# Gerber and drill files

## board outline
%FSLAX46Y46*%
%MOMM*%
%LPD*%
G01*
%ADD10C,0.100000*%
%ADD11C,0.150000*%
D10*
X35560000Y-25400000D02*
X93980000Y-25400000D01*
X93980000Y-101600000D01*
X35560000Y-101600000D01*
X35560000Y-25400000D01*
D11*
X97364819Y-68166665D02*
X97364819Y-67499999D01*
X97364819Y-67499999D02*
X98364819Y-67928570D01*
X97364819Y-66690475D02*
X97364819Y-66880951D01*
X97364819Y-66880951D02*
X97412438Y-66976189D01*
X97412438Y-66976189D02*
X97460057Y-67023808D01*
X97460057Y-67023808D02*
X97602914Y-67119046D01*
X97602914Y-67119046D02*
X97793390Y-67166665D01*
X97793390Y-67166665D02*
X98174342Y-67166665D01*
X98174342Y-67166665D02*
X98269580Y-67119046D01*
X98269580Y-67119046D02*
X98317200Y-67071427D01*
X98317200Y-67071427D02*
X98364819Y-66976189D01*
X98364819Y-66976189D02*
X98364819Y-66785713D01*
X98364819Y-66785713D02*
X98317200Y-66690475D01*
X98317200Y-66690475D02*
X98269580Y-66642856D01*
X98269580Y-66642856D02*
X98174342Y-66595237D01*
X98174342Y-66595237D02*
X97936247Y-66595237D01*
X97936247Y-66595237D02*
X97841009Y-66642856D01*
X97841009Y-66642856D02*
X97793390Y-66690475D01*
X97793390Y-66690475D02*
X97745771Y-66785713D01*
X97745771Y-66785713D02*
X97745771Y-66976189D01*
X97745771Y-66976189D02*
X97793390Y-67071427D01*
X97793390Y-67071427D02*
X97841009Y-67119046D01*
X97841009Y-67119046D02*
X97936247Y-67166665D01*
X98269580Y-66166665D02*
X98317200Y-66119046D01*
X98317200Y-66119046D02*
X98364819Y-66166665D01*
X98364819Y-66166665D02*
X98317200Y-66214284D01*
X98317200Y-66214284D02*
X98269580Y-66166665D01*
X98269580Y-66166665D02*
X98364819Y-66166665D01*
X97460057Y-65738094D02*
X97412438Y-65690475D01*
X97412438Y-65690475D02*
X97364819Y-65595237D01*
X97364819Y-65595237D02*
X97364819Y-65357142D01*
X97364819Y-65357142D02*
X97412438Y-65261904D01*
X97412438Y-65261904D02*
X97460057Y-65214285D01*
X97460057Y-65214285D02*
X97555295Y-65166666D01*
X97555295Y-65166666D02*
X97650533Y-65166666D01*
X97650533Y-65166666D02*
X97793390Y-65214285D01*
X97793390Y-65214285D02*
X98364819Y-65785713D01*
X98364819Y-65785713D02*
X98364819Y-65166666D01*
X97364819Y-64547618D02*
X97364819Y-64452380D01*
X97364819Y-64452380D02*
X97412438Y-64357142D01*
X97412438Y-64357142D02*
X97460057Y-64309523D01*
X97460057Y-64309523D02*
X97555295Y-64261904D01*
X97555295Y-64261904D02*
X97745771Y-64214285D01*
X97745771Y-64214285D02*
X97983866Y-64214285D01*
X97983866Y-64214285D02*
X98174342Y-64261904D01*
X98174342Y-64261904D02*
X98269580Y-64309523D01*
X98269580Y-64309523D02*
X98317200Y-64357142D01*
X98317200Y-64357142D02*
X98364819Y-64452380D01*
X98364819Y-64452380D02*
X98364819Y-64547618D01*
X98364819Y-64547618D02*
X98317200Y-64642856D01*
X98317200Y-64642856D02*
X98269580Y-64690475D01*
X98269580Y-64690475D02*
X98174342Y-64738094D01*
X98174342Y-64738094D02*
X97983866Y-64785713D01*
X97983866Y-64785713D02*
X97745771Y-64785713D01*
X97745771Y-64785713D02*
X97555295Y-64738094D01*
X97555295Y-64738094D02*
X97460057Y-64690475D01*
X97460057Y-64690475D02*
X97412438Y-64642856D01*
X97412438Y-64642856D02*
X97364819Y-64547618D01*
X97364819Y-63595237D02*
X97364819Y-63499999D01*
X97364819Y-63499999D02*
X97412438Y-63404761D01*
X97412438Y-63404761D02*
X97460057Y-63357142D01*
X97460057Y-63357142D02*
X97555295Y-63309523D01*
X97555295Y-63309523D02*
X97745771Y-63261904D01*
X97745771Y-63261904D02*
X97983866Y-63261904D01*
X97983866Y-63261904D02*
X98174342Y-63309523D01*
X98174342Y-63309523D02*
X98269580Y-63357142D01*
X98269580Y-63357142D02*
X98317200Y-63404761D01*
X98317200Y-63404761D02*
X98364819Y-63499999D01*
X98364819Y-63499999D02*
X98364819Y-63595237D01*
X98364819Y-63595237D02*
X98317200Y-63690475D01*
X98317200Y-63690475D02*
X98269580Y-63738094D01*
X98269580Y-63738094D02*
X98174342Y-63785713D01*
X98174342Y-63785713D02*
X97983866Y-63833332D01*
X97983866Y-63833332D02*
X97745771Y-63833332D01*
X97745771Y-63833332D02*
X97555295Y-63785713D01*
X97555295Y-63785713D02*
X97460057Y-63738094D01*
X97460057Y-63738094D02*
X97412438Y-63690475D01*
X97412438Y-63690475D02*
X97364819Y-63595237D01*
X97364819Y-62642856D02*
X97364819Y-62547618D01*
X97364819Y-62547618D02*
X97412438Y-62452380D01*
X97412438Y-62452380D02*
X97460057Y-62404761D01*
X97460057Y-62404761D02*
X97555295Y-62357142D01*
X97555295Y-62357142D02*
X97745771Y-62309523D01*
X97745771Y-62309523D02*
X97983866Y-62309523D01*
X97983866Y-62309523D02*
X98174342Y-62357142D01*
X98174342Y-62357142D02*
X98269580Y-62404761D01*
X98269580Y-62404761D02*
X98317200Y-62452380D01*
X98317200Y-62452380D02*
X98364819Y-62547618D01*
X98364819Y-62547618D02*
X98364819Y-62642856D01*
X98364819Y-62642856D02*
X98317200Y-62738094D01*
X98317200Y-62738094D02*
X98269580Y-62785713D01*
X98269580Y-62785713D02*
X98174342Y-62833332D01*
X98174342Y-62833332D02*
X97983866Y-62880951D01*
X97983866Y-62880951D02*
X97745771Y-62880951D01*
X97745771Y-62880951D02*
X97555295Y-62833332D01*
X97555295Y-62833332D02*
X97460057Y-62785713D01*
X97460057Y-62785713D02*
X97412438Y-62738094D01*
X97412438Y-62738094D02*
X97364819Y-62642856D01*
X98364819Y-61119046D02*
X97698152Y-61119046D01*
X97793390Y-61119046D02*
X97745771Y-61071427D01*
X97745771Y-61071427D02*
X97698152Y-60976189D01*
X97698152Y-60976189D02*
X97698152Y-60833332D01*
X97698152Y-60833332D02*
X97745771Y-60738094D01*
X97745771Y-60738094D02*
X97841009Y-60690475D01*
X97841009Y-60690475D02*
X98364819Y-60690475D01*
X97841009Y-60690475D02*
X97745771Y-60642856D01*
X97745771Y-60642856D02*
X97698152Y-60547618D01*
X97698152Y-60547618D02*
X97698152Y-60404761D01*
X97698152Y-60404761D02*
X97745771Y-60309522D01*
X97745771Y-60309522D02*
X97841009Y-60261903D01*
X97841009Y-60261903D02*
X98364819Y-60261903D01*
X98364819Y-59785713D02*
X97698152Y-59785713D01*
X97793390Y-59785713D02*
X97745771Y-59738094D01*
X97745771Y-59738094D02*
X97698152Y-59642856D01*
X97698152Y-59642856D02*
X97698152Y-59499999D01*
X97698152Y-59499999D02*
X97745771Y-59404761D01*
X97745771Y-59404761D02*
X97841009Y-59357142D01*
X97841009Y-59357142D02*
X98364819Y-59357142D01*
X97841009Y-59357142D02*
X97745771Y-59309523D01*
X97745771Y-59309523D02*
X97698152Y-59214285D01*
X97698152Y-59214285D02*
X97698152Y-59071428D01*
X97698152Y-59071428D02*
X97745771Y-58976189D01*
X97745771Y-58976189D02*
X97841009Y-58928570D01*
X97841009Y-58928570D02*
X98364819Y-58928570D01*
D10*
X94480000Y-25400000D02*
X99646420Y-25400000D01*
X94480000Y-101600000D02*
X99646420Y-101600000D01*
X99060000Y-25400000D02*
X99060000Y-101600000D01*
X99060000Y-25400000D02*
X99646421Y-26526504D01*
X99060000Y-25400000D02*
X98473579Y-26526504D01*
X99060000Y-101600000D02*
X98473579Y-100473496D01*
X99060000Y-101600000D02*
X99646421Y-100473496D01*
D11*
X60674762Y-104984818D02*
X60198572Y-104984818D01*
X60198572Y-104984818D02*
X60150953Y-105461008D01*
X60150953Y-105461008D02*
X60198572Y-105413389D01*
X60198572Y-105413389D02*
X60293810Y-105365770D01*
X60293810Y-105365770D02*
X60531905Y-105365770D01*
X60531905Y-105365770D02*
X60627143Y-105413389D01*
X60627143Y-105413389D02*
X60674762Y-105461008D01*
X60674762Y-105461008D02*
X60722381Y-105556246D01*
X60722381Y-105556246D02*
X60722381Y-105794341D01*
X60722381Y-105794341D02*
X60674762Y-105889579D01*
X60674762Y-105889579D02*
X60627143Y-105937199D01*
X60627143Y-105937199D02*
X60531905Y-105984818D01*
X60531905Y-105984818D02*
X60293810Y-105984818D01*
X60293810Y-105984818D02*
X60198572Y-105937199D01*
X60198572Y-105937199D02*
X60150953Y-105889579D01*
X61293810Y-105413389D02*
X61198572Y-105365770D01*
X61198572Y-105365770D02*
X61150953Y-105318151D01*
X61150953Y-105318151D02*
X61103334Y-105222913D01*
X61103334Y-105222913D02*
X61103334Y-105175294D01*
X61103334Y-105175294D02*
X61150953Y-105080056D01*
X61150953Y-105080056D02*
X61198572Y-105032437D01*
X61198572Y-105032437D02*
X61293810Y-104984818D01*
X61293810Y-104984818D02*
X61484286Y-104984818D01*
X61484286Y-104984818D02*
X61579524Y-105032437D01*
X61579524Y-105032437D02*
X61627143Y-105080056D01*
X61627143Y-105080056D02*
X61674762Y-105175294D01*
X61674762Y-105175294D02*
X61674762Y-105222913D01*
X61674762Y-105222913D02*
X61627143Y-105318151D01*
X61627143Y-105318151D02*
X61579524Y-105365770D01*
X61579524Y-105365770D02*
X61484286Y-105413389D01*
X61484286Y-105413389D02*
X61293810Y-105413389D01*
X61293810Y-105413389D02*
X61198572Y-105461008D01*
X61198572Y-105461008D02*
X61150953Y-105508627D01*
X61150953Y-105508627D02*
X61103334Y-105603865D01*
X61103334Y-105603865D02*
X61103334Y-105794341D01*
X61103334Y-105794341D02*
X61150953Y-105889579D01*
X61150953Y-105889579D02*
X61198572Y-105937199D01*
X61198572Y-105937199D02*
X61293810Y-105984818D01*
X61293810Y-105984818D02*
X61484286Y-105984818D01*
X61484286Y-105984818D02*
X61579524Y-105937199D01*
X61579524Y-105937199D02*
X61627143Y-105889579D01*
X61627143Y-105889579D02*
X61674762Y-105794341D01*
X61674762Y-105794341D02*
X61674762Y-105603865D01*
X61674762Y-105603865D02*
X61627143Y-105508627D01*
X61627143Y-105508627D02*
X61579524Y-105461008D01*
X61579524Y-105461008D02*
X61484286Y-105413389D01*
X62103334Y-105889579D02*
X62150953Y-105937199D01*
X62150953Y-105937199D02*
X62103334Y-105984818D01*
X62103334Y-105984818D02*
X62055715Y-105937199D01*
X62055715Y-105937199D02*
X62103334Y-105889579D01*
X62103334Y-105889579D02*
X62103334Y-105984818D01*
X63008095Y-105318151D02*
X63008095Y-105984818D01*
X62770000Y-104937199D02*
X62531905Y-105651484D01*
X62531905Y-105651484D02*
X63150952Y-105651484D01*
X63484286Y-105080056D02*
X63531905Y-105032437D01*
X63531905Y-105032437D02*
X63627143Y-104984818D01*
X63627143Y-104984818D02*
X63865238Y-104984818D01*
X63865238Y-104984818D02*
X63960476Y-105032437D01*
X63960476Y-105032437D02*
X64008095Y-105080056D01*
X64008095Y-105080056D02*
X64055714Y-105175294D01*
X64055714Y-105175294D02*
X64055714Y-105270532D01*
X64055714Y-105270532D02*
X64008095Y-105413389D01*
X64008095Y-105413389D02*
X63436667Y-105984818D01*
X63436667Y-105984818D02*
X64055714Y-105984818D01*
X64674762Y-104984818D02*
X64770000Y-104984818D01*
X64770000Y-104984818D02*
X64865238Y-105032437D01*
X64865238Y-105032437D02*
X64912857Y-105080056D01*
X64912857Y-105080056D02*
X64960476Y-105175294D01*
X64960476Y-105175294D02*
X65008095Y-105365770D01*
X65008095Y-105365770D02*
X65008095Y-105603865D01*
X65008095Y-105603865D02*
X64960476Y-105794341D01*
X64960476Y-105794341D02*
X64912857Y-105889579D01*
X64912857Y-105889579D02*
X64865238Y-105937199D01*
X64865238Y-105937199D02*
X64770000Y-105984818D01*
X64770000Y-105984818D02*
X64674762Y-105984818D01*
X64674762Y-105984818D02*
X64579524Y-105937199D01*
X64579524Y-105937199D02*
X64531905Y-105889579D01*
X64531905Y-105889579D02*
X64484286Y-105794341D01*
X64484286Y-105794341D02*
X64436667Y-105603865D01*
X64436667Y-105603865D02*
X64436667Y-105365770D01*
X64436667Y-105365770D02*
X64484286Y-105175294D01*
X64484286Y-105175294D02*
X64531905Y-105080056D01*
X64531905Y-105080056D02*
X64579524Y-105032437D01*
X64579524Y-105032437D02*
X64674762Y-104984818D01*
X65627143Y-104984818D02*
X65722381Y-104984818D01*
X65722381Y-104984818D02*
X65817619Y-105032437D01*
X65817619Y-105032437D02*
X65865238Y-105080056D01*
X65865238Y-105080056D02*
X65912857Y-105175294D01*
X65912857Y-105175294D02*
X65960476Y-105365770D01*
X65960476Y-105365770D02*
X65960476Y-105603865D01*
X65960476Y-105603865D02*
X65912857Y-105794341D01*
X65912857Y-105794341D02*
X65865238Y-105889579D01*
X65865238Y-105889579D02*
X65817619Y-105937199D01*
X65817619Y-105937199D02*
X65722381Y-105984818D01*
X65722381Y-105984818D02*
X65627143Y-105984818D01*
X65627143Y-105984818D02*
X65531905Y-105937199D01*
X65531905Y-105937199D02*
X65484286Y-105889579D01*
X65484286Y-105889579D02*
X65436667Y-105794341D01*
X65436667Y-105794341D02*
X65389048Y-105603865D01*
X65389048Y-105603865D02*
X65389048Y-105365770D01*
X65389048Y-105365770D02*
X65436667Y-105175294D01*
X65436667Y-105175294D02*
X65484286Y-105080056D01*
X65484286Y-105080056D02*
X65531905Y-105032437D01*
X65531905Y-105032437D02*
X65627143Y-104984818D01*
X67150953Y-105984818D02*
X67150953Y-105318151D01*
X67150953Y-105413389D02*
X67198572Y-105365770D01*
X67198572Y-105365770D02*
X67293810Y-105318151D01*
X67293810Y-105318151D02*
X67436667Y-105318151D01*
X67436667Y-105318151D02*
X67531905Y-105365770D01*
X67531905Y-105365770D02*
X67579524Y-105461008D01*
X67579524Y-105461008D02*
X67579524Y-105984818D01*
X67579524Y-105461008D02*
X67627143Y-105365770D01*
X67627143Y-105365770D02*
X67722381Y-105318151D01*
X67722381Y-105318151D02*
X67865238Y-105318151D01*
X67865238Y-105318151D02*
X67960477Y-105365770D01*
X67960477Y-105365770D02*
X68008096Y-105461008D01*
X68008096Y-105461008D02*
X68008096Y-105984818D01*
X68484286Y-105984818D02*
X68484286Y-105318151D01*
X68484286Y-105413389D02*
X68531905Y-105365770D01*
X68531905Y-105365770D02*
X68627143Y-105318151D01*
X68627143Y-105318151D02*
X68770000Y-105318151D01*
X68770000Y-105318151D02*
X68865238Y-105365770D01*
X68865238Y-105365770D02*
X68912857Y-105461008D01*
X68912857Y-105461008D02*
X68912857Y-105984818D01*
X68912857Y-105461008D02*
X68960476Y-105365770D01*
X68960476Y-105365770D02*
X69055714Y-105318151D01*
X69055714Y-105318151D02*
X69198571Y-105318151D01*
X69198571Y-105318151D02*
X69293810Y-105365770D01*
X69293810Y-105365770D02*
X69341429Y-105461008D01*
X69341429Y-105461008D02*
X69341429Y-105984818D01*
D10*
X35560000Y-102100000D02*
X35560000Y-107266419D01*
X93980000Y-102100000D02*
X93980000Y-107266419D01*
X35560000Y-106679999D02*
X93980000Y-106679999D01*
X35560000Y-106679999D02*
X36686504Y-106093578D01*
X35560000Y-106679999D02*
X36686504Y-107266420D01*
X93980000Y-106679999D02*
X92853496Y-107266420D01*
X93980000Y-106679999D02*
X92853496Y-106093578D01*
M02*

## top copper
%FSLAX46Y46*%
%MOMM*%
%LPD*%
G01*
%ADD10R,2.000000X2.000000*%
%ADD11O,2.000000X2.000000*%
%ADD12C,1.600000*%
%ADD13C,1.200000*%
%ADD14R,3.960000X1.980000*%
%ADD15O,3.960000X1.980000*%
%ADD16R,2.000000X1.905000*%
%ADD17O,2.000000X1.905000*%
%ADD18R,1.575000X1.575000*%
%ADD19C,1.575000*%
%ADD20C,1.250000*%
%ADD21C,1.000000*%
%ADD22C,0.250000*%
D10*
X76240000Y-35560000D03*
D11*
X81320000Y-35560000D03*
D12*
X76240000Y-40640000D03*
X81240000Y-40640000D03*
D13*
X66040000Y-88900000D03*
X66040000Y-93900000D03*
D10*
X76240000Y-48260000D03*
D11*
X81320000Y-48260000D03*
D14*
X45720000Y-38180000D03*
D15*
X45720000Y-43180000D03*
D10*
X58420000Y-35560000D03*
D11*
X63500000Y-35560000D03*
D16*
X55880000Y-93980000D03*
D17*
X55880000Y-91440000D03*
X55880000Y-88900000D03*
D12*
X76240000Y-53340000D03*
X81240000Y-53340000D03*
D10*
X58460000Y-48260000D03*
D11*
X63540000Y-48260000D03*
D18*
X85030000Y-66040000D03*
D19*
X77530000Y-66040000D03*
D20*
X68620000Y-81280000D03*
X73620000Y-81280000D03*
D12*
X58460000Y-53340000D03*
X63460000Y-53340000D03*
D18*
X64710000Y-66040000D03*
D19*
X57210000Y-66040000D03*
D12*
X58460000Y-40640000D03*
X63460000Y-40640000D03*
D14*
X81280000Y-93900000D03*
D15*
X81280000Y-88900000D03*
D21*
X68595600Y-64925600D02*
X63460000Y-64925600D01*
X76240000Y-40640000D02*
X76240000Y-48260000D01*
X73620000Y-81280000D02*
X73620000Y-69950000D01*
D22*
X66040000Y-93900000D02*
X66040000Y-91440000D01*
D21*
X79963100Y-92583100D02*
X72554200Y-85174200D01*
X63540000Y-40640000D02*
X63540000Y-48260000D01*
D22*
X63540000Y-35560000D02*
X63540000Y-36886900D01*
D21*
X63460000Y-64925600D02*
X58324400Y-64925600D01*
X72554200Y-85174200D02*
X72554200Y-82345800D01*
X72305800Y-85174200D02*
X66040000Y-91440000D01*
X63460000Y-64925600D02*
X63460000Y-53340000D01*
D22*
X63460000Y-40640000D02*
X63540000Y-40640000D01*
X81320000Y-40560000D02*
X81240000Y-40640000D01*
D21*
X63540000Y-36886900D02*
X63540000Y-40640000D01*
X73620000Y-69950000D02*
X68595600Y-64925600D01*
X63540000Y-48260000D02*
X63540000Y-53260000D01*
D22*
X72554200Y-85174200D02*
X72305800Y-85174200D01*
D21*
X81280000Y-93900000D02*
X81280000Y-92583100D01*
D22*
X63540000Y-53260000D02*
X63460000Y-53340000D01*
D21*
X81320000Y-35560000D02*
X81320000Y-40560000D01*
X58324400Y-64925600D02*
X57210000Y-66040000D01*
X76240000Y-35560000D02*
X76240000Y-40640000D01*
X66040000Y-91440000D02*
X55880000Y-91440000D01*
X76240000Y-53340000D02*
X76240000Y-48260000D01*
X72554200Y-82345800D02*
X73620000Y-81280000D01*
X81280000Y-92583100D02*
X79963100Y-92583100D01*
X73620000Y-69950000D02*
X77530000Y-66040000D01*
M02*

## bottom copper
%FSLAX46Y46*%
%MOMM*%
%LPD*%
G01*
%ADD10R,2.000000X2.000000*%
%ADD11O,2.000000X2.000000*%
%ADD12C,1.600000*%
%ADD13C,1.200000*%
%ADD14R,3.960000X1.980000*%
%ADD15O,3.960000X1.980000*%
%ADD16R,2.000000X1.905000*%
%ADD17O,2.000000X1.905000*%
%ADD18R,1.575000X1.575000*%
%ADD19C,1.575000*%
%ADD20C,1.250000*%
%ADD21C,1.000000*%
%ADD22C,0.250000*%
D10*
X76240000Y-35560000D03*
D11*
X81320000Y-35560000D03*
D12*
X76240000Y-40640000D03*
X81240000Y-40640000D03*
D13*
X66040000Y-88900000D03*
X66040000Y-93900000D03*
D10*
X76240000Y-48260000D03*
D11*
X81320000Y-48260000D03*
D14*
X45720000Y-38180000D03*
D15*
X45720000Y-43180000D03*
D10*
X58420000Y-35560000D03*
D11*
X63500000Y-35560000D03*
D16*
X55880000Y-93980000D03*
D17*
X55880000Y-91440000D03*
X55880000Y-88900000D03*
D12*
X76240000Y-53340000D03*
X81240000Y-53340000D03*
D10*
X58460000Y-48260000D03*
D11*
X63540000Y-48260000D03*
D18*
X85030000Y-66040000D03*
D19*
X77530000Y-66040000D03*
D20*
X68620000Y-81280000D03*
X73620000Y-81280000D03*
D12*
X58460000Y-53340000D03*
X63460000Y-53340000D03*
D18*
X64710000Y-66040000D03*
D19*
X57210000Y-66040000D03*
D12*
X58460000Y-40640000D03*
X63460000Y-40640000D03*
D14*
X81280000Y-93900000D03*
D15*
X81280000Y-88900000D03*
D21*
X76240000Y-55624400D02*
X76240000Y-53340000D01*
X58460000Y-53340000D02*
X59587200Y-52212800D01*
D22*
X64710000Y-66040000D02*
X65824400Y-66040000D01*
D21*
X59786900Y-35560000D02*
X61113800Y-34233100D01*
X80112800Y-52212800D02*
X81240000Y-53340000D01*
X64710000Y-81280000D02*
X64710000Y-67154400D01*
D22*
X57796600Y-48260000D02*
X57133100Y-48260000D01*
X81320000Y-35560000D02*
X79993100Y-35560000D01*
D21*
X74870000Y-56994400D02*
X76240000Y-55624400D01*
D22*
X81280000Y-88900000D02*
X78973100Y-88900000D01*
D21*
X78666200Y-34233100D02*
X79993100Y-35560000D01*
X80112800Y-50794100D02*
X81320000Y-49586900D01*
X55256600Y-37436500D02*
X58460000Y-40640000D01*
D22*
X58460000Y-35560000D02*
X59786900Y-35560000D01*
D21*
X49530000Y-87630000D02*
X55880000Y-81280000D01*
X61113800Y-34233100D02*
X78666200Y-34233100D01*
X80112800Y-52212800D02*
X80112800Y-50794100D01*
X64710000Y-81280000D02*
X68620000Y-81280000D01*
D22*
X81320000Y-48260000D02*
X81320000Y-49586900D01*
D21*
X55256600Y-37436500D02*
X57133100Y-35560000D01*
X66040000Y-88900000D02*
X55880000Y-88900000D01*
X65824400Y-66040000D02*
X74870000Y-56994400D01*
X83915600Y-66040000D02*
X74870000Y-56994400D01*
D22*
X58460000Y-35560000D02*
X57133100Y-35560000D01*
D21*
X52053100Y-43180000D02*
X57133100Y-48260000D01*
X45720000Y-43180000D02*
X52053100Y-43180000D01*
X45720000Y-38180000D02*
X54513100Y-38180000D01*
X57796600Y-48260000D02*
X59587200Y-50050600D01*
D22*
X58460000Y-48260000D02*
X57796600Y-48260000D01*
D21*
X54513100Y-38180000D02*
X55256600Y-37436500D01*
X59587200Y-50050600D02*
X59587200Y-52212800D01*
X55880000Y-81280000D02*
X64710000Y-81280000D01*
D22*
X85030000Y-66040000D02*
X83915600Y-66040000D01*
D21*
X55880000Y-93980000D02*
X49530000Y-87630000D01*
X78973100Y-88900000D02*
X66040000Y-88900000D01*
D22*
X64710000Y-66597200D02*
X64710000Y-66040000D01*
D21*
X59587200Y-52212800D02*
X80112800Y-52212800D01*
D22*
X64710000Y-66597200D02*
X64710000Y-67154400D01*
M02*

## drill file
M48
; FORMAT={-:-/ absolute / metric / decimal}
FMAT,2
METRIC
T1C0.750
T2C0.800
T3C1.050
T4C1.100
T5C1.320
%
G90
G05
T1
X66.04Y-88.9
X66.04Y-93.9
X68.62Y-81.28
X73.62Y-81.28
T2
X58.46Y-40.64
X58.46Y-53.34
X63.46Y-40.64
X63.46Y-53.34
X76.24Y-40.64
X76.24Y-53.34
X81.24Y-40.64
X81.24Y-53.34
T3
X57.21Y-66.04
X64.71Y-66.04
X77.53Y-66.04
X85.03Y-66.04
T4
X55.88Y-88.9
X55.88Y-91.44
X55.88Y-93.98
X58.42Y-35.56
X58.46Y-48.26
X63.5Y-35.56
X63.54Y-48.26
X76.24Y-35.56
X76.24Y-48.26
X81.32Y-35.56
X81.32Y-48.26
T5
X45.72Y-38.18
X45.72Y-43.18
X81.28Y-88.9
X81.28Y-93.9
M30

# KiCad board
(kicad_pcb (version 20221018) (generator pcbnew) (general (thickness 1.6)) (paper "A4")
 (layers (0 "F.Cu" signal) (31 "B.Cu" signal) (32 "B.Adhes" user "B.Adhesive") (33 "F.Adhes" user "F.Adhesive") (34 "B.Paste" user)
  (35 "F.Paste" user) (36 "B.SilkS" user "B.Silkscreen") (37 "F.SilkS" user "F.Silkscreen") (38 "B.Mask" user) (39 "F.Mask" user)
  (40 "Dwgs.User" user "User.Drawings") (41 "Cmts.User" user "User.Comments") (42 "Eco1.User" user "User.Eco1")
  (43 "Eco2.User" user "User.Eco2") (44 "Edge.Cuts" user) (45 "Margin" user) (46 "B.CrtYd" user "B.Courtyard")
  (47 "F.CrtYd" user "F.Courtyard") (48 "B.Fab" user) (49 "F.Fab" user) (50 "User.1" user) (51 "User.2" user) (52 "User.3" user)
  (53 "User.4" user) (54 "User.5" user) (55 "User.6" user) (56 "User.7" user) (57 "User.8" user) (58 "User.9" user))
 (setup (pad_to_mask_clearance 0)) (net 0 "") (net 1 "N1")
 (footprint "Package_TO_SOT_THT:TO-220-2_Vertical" (layer "F.Cu") (at 76.24 35.56)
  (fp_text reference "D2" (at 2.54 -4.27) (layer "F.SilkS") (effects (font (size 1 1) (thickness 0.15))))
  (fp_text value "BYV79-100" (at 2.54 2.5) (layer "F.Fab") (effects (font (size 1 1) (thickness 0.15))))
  (pad "1" thru_hole rect (at 0 0) (size 2 2) (drill 1.1) (layers "*.Cu" "*.Mask") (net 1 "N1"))
  (pad "2" thru_hole oval (at 5.08 0) (size 2 2) (drill 1.1) (layers "*.Cu" "*.Mask") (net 1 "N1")))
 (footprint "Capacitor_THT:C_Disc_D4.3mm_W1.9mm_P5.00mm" (layer "F.Cu") (at 76.24 40.64)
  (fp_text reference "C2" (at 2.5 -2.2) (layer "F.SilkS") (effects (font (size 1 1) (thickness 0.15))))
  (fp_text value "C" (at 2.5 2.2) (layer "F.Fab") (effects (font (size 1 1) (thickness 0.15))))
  (pad "1" thru_hole circle (at 0 0) (size 1.6 1.6) (drill 0.8) (layers "*.Cu" "*.Mask") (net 1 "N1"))
  (pad "2" thru_hole circle (at 5 0) (size 1.6 1.6) (drill 0.8) (layers "*.Cu" "*.Mask") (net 1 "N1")))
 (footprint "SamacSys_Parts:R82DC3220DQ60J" (layer "F.Cu") (at 66.04 88.9 -90)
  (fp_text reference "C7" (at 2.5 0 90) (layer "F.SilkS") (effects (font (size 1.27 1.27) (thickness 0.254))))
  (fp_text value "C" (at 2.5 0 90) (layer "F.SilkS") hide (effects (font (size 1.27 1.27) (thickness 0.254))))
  (pad "1" thru_hole circle (at 0 0 270) (size 1.2 1.2) (drill 0.75) (layers "*.Cu" "*.Mask") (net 1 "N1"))
  (pad "2" thru_hole circle (at 5 0 270) (size 1.2 1.2) (drill 0.75) (layers "*.Cu" "*.Mask") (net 1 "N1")))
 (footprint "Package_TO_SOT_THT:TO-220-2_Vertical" (layer "F.Cu") (at 76.24 48.26)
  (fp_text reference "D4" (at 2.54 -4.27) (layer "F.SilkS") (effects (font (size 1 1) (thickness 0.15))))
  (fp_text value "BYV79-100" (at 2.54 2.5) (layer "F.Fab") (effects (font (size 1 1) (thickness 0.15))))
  (pad "1" thru_hole rect (at 0 0) (size 2 2) (drill 1.1) (layers "*.Cu" "*.Mask") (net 1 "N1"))
  (pad "2" thru_hole oval (at 5.08 0) (size 2 2) (drill 1.1) (layers "*.Cu" "*.Mask") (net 1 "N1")))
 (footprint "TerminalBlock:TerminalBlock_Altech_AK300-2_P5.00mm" (layer "F.Cu") (at 45.72 38.18 -90)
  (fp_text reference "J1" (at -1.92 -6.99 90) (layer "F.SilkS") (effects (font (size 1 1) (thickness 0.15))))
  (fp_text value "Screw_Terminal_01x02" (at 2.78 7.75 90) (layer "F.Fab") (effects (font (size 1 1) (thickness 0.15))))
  (pad "1" thru_hole rect (at 0 0 270) (size 1.98 3.96) (drill 1.32) (layers "*.Cu" "*.Mask") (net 1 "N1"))
  (pad "2" thru_hole oval (at 5 0 270) (size 1.98 3.96) (drill 1.32) (layers "*.Cu" "*.Mask") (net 1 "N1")))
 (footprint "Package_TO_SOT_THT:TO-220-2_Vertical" (layer "F.Cu") (at 58.42 35.56)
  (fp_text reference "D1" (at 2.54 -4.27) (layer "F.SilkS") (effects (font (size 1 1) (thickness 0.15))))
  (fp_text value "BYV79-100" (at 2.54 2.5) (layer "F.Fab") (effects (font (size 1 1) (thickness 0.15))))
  (pad "1" thru_hole rect (at 0 0) (size 2 2) (drill 1.1) (layers "*.Cu" "*.Mask") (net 1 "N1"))
  (pad "2" thru_hole oval (at 5.08 0) (size 2 2) (drill 1.1) (layers "*.Cu" "*.Mask") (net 1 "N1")))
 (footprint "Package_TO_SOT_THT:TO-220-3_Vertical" (layer "F.Cu") (at 55.88 93.98 90)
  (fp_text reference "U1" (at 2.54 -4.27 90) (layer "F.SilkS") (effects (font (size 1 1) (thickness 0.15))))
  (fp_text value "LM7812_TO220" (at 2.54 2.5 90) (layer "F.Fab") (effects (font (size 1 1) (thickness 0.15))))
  (pad "1" thru_hole rect (at 0 0 90) (size 1.905 2) (drill 1.1) (layers "*.Cu" "*.Mask") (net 1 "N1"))
  (pad "2" thru_hole oval (at 2.54 0 90) (size 1.905 2) (drill 1.1) (layers "*.Cu" "*.Mask") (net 1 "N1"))
  (pad "3" thru_hole oval (at 5.08 0 90) (size 1.905 2) (drill 1.1) (layers "*.Cu" "*.Mask") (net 1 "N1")))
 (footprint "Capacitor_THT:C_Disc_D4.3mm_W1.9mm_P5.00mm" (layer "F.Cu") (at 76.24 53.34)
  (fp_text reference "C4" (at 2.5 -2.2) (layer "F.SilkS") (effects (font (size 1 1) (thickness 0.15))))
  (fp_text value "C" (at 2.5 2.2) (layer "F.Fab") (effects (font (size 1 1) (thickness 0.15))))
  (pad "1" thru_hole circle (at 0 0) (size 1.6 1.6) (drill 0.8) (layers "*.Cu" "*.Mask") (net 1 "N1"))
  (pad "2" thru_hole circle (at 5 0) (size 1.6 1.6) (drill 0.8) (layers "*.Cu" "*.Mask") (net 1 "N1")))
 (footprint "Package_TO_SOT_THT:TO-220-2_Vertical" (layer "F.Cu") (at 58.46 48.26)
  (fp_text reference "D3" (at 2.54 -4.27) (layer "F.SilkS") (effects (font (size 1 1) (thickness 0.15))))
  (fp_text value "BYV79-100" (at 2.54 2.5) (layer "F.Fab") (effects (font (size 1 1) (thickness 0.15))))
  (pad "1" thru_hole rect (at 0 0) (size 2 2) (drill 1.1) (layers "*.Cu" "*.Mask") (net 1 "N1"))
  (pad "2" thru_hole oval (at 5.08 0) (size 2 2) (drill 1.1) (layers "*.Cu" "*.Mask") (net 1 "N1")))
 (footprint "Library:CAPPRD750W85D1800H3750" (layer "F.Cu") (at 85.03 66.04 180)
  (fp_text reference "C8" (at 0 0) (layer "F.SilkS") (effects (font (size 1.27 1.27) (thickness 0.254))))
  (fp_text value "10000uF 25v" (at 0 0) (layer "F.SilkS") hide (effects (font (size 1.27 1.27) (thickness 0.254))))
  (pad "1" thru_hole rect (at 0 0 180) (size 1.575 1.575) (drill 1.05) (layers "*.Cu" "*.Mask") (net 1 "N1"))
  (pad "2" thru_hole circle (at 7.5 0 180) (size 1.575 1.575) (drill 1.05) (layers "*.Cu" "*.Mask") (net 1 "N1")))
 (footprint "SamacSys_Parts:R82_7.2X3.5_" (layer "F.Cu") (at 71.12 81.28)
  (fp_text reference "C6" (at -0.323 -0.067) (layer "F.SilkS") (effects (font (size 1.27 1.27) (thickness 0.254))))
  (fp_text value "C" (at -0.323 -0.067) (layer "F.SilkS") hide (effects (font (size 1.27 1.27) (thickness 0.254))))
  (pad "1" thru_hole circle (at -2.5 0) (size 1.25 1.25) (drill 0.75) (layers "*.Cu" "*.Mask") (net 1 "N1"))
  (pad "2" thru_hole circle (at 2.5 0) (size 1.25 1.25) (drill 0.75) (layers "*.Cu" "*.Mask") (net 1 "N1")))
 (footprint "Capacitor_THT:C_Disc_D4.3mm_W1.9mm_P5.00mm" (layer "F.Cu") (at 58.46 53.34)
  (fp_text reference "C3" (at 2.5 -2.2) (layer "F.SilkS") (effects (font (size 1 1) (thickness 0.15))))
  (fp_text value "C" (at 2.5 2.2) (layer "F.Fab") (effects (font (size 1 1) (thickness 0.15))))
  (pad "1" thru_hole circle (at 0 0) (size 1.6 1.6) (drill 0.8) (layers "*.Cu" "*.Mask") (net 1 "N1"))
  (pad "2" thru_hole circle (at 5 0) (size 1.6 1.6) (drill 0.8) (layers "*.Cu" "*.Mask") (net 1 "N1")))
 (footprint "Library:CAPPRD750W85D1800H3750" (layer "F.Cu") (at 64.71 66.04 180)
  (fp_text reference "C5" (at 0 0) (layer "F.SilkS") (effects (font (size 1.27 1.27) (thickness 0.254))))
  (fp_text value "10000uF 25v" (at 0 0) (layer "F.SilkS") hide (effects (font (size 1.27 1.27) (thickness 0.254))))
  (pad "1" thru_hole rect (at 0 0 180) (size 1.575 1.575) (drill 1.05) (layers "*.Cu" "*.Mask") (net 1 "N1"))
  (pad "2" thru_hole circle (at 7.5 0 180) (size 1.575 1.575) (drill 1.05) (layers "*.Cu" "*.Mask") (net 1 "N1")))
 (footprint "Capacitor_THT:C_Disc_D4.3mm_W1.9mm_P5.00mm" (layer "F.Cu") (at 58.46 40.64)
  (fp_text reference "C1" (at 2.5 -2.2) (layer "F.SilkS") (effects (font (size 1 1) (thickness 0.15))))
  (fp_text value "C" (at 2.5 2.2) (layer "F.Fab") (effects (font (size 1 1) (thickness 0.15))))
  (pad "1" thru_hole circle (at 0 0) (size 1.6 1.6) (drill 0.8) (layers "*.Cu" "*.Mask") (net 1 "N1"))
  (pad "2" thru_hole circle (at 5 0) (size 1.6 1.6) (drill 0.8) (layers "*.Cu" "*.Mask") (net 1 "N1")))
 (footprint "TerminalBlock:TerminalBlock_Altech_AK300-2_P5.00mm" (layer "F.Cu") (at 81.28 93.9 90)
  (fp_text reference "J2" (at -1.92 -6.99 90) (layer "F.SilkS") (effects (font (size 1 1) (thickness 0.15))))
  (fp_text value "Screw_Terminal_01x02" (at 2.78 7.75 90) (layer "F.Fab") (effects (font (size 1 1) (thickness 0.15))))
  (pad "1" thru_hole rect (at 0 0 90) (size 1.98 3.96) (drill 1.32) (layers "*.Cu" "*.Mask") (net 1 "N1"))
  (pad "2" thru_hole oval (at 5 0 90) (size 1.98 3.96) (drill 1.32) (layers "*.Cu" "*.Mask") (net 1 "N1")))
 (gr_rect (start 35.56 25.4) (end 93.98 101.6) (stroke (width 0.1) (type default)) (fill none) (layer "Edge.Cuts"))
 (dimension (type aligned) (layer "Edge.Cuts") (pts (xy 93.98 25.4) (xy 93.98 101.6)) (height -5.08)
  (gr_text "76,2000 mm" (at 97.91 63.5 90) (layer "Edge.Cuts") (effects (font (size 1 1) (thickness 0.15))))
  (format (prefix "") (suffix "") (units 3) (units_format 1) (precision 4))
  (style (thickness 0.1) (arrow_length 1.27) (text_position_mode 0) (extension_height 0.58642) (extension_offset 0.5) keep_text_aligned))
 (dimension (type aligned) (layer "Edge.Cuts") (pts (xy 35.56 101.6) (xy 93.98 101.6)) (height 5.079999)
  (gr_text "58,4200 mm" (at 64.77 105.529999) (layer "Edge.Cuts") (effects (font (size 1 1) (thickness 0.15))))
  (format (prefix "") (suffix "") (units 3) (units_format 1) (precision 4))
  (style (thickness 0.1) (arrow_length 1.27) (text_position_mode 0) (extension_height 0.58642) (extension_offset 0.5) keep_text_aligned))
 (segment (start 68.5956 64.9256) (end 63.46 64.9256) (width 1) (layer "F.Cu") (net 1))
 (segment (start 76.24 40.64) (end 76.24 48.26) (width 1) (layer "F.Cu") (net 1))
 (segment (start 73.62 81.28) (end 73.62 69.95) (width 1) (layer "F.Cu") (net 1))
 (segment (start 66.04 93.9) (end 66.04 91.44) (width 0.25) (layer "F.Cu") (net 1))
 (segment (start 79.9631 92.5831) (end 72.5542 85.1742) (width 1) (layer "F.Cu") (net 1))
 (segment (start 63.54 40.64) (end 63.54 48.26) (width 1) (layer "F.Cu") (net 1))
 (segment (start 63.54 35.56) (end 63.54 36.8869) (width 0.25) (layer "F.Cu") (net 1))
 (segment (start 63.46 64.9256) (end 58.3244 64.9256) (width 1) (layer "F.Cu") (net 1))
 (segment (start 72.5542 85.1742) (end 72.5542 82.3458) (width 1) (layer "F.Cu") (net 1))
 (segment (start 72.3058 85.1742) (end 66.04 91.44) (width 1) (layer "F.Cu") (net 1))
 (segment (start 63.46 64.9256) (end 63.46 53.34) (width 1) (layer "F.Cu") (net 1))
 (segment (start 63.46 40.64) (end 63.54 40.64) (width 0.25) (layer "F.Cu") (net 1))
 (segment (start 81.32 40.56) (end 81.24 40.64) (width 0.25) (layer "F.Cu") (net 1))
 (segment (start 63.54 36.8869) (end 63.54 40.64) (width 1) (layer "F.Cu") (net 1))
 (segment (start 73.62 69.95) (end 68.5956 64.9256) (width 1) (layer "F.Cu") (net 1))
 (segment (start 63.54 48.26) (end 63.54 53.26) (width 1) (layer "F.Cu") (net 1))
 (segment (start 72.5542 85.1742) (end 72.3058 85.1742) (width 0.25) (layer "F.Cu") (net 1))
 (segment (start 81.28 93.9) (end 81.28 92.5831) (width 1) (layer "F.Cu") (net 1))
 (segment (start 63.54 53.26) (end 63.46 53.34) (width 0.25) (layer "F.Cu") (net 1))
 (segment (start 81.32 35.56) (end 81.32 40.56) (width 1) (layer "F.Cu") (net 1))
 (segment (start 58.3244 64.9256) (end 57.21 66.04) (width 1) (layer "F.Cu") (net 1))
 (segment (start 76.24 35.56) (end 76.24 40.64) (width 1) (layer "F.Cu") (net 1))
 (segment (start 66.04 91.44) (end 55.88 91.44) (width 1) (layer "F.Cu") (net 1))
 (segment (start 76.24 53.34) (end 76.24 48.26) (width 1) (layer "F.Cu") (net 1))
 (segment (start 72.5542 82.3458) (end 73.62 81.28) (width 1) (layer "F.Cu") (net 1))
 (segment (start 81.28 92.5831) (end 79.9631 92.5831) (width 1) (layer "F.Cu") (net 1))
 (segment (start 73.62 69.95) (end 77.53 66.04) (width 1) (layer "F.Cu") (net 1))
 (segment (start 76.24 55.6244) (end 76.24 53.34) (width 1) (layer "B.Cu") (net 1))
 (segment (start 58.46 53.34) (end 59.5872 52.2128) (width 1) (layer "B.Cu") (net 1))
 (segment (start 64.71 66.04) (end 65.8244 66.04) (width 0.25) (layer "B.Cu") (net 1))
 (segment (start 59.7869 35.56) (end 61.1138 34.2331) (width 1) (layer "B.Cu") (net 1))
 (segment (start 80.1128 52.2128) (end 81.24 53.34) (width 1) (layer "B.Cu") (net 1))
 (segment (start 64.71 81.28) (end 64.71 67.1544) (width 1) (layer "B.Cu") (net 1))
 (segment (start 57.7966 48.26) (end 57.1331 48.26) (width 0.25) (layer "B.Cu") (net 1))
 (segment (start 81.32 35.56) (end 79.9931 35.56) (width 0.25) (layer "B.Cu") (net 1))
 (segment (start 74.87 56.9944) (end 76.24 55.6244) (width 1) (layer "B.Cu") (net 1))
 (segment (start 81.28 88.9) (end 78.9731 88.9) (width 0.25) (layer "B.Cu") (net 1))
 (segment (start 78.6662 34.2331) (end 79.9931 35.56) (width 1) (layer "B.Cu") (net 1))
 (segment (start 80.1128 50.7941) (end 81.32 49.5869) (width 1) (layer "B.Cu") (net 1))
 (segment (start 55.2566 37.4365) (end 58.46 40.64) (width 1) (layer "B.Cu") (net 1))
 (segment (start 58.46 35.56) (end 59.7869 35.56) (width 0.25) (layer "B.Cu") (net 1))
 (segment (start 49.53 87.63) (end 55.88 81.28) (width 1) (layer "B.Cu") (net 1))
 (segment (start 61.1138 34.2331) (end 78.6662 34.2331) (width 1) (layer "B.Cu") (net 1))
 (segment (start 80.1128 52.2128) (end 80.1128 50.7941) (width 1) (layer "B.Cu") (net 1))
 (segment (start 64.71 81.28) (end 68.62 81.28) (width 1) (layer "B.Cu") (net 1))
 (segment (start 81.32 48.26) (end 81.32 49.5869) (width 0.25) (layer "B.Cu") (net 1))
 (segment (start 55.2566 37.4365) (end 57.1331 35.56) (width 1) (layer "B.Cu") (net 1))
 (segment (start 66.04 88.9) (end 55.88 88.9) (width 1) (layer "B.Cu") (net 1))
 (segment (start 65.8244 66.04) (end 74.87 56.9944) (width 1) (layer "B.Cu") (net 1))
 (segment (start 83.9156 66.04) (end 74.87 56.9944) (width 1) (layer "B.Cu") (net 1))
 (segment (start 58.46 35.56) (end 57.1331 35.56) (width 0.25) (layer "B.Cu") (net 1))
 (segment (start 52.0531 43.18) (end 57.1331 48.26) (width 1) (layer "B.Cu") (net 1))
 (segment (start 45.72 43.18) (end 52.0531 43.18) (width 1) (layer "B.Cu") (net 1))
 (segment (start 45.72 38.18) (end 54.5131 38.18) (width 1) (layer "B.Cu") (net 1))
 (segment (start 57.7966 48.26) (end 59.5872 50.0506) (width 1) (layer "B.Cu") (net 1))
 (segment (start 58.46 48.26) (end 57.7966 48.26) (width 0.25) (layer "B.Cu") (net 1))
 (segment (start 54.5131 38.18) (end 55.2566 37.4365) (width 1) (layer "B.Cu") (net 1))
 (segment (start 59.5872 50.0506) (end 59.5872 52.2128) (width 1) (layer "B.Cu") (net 1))
 (segment (start 55.88 81.28) (end 64.71 81.28) (width 1) (layer "B.Cu") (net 1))
 (segment (start 85.03 66.04) (end 83.9156 66.04) (width 0.25) (layer "B.Cu") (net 1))
 (segment (start 55.88 93.98) (end 49.53 87.63) (width 1) (layer "B.Cu") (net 1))
 (segment (start 78.9731 88.9) (end 66.04 88.9) (width 1) (layer "B.Cu") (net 1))
 (segment (start 64.71 66.5972) (end 64.71 66.04) (width 0.25) (layer "B.Cu") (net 1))
 (segment (start 59.5872 52.2128) (end 80.1128 52.2128) (width 1) (layer "B.Cu") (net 1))
 (segment (start 64.71 66.5972) (end 64.71 67.1544) (width 0.25) (layer "B.Cu") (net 1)))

